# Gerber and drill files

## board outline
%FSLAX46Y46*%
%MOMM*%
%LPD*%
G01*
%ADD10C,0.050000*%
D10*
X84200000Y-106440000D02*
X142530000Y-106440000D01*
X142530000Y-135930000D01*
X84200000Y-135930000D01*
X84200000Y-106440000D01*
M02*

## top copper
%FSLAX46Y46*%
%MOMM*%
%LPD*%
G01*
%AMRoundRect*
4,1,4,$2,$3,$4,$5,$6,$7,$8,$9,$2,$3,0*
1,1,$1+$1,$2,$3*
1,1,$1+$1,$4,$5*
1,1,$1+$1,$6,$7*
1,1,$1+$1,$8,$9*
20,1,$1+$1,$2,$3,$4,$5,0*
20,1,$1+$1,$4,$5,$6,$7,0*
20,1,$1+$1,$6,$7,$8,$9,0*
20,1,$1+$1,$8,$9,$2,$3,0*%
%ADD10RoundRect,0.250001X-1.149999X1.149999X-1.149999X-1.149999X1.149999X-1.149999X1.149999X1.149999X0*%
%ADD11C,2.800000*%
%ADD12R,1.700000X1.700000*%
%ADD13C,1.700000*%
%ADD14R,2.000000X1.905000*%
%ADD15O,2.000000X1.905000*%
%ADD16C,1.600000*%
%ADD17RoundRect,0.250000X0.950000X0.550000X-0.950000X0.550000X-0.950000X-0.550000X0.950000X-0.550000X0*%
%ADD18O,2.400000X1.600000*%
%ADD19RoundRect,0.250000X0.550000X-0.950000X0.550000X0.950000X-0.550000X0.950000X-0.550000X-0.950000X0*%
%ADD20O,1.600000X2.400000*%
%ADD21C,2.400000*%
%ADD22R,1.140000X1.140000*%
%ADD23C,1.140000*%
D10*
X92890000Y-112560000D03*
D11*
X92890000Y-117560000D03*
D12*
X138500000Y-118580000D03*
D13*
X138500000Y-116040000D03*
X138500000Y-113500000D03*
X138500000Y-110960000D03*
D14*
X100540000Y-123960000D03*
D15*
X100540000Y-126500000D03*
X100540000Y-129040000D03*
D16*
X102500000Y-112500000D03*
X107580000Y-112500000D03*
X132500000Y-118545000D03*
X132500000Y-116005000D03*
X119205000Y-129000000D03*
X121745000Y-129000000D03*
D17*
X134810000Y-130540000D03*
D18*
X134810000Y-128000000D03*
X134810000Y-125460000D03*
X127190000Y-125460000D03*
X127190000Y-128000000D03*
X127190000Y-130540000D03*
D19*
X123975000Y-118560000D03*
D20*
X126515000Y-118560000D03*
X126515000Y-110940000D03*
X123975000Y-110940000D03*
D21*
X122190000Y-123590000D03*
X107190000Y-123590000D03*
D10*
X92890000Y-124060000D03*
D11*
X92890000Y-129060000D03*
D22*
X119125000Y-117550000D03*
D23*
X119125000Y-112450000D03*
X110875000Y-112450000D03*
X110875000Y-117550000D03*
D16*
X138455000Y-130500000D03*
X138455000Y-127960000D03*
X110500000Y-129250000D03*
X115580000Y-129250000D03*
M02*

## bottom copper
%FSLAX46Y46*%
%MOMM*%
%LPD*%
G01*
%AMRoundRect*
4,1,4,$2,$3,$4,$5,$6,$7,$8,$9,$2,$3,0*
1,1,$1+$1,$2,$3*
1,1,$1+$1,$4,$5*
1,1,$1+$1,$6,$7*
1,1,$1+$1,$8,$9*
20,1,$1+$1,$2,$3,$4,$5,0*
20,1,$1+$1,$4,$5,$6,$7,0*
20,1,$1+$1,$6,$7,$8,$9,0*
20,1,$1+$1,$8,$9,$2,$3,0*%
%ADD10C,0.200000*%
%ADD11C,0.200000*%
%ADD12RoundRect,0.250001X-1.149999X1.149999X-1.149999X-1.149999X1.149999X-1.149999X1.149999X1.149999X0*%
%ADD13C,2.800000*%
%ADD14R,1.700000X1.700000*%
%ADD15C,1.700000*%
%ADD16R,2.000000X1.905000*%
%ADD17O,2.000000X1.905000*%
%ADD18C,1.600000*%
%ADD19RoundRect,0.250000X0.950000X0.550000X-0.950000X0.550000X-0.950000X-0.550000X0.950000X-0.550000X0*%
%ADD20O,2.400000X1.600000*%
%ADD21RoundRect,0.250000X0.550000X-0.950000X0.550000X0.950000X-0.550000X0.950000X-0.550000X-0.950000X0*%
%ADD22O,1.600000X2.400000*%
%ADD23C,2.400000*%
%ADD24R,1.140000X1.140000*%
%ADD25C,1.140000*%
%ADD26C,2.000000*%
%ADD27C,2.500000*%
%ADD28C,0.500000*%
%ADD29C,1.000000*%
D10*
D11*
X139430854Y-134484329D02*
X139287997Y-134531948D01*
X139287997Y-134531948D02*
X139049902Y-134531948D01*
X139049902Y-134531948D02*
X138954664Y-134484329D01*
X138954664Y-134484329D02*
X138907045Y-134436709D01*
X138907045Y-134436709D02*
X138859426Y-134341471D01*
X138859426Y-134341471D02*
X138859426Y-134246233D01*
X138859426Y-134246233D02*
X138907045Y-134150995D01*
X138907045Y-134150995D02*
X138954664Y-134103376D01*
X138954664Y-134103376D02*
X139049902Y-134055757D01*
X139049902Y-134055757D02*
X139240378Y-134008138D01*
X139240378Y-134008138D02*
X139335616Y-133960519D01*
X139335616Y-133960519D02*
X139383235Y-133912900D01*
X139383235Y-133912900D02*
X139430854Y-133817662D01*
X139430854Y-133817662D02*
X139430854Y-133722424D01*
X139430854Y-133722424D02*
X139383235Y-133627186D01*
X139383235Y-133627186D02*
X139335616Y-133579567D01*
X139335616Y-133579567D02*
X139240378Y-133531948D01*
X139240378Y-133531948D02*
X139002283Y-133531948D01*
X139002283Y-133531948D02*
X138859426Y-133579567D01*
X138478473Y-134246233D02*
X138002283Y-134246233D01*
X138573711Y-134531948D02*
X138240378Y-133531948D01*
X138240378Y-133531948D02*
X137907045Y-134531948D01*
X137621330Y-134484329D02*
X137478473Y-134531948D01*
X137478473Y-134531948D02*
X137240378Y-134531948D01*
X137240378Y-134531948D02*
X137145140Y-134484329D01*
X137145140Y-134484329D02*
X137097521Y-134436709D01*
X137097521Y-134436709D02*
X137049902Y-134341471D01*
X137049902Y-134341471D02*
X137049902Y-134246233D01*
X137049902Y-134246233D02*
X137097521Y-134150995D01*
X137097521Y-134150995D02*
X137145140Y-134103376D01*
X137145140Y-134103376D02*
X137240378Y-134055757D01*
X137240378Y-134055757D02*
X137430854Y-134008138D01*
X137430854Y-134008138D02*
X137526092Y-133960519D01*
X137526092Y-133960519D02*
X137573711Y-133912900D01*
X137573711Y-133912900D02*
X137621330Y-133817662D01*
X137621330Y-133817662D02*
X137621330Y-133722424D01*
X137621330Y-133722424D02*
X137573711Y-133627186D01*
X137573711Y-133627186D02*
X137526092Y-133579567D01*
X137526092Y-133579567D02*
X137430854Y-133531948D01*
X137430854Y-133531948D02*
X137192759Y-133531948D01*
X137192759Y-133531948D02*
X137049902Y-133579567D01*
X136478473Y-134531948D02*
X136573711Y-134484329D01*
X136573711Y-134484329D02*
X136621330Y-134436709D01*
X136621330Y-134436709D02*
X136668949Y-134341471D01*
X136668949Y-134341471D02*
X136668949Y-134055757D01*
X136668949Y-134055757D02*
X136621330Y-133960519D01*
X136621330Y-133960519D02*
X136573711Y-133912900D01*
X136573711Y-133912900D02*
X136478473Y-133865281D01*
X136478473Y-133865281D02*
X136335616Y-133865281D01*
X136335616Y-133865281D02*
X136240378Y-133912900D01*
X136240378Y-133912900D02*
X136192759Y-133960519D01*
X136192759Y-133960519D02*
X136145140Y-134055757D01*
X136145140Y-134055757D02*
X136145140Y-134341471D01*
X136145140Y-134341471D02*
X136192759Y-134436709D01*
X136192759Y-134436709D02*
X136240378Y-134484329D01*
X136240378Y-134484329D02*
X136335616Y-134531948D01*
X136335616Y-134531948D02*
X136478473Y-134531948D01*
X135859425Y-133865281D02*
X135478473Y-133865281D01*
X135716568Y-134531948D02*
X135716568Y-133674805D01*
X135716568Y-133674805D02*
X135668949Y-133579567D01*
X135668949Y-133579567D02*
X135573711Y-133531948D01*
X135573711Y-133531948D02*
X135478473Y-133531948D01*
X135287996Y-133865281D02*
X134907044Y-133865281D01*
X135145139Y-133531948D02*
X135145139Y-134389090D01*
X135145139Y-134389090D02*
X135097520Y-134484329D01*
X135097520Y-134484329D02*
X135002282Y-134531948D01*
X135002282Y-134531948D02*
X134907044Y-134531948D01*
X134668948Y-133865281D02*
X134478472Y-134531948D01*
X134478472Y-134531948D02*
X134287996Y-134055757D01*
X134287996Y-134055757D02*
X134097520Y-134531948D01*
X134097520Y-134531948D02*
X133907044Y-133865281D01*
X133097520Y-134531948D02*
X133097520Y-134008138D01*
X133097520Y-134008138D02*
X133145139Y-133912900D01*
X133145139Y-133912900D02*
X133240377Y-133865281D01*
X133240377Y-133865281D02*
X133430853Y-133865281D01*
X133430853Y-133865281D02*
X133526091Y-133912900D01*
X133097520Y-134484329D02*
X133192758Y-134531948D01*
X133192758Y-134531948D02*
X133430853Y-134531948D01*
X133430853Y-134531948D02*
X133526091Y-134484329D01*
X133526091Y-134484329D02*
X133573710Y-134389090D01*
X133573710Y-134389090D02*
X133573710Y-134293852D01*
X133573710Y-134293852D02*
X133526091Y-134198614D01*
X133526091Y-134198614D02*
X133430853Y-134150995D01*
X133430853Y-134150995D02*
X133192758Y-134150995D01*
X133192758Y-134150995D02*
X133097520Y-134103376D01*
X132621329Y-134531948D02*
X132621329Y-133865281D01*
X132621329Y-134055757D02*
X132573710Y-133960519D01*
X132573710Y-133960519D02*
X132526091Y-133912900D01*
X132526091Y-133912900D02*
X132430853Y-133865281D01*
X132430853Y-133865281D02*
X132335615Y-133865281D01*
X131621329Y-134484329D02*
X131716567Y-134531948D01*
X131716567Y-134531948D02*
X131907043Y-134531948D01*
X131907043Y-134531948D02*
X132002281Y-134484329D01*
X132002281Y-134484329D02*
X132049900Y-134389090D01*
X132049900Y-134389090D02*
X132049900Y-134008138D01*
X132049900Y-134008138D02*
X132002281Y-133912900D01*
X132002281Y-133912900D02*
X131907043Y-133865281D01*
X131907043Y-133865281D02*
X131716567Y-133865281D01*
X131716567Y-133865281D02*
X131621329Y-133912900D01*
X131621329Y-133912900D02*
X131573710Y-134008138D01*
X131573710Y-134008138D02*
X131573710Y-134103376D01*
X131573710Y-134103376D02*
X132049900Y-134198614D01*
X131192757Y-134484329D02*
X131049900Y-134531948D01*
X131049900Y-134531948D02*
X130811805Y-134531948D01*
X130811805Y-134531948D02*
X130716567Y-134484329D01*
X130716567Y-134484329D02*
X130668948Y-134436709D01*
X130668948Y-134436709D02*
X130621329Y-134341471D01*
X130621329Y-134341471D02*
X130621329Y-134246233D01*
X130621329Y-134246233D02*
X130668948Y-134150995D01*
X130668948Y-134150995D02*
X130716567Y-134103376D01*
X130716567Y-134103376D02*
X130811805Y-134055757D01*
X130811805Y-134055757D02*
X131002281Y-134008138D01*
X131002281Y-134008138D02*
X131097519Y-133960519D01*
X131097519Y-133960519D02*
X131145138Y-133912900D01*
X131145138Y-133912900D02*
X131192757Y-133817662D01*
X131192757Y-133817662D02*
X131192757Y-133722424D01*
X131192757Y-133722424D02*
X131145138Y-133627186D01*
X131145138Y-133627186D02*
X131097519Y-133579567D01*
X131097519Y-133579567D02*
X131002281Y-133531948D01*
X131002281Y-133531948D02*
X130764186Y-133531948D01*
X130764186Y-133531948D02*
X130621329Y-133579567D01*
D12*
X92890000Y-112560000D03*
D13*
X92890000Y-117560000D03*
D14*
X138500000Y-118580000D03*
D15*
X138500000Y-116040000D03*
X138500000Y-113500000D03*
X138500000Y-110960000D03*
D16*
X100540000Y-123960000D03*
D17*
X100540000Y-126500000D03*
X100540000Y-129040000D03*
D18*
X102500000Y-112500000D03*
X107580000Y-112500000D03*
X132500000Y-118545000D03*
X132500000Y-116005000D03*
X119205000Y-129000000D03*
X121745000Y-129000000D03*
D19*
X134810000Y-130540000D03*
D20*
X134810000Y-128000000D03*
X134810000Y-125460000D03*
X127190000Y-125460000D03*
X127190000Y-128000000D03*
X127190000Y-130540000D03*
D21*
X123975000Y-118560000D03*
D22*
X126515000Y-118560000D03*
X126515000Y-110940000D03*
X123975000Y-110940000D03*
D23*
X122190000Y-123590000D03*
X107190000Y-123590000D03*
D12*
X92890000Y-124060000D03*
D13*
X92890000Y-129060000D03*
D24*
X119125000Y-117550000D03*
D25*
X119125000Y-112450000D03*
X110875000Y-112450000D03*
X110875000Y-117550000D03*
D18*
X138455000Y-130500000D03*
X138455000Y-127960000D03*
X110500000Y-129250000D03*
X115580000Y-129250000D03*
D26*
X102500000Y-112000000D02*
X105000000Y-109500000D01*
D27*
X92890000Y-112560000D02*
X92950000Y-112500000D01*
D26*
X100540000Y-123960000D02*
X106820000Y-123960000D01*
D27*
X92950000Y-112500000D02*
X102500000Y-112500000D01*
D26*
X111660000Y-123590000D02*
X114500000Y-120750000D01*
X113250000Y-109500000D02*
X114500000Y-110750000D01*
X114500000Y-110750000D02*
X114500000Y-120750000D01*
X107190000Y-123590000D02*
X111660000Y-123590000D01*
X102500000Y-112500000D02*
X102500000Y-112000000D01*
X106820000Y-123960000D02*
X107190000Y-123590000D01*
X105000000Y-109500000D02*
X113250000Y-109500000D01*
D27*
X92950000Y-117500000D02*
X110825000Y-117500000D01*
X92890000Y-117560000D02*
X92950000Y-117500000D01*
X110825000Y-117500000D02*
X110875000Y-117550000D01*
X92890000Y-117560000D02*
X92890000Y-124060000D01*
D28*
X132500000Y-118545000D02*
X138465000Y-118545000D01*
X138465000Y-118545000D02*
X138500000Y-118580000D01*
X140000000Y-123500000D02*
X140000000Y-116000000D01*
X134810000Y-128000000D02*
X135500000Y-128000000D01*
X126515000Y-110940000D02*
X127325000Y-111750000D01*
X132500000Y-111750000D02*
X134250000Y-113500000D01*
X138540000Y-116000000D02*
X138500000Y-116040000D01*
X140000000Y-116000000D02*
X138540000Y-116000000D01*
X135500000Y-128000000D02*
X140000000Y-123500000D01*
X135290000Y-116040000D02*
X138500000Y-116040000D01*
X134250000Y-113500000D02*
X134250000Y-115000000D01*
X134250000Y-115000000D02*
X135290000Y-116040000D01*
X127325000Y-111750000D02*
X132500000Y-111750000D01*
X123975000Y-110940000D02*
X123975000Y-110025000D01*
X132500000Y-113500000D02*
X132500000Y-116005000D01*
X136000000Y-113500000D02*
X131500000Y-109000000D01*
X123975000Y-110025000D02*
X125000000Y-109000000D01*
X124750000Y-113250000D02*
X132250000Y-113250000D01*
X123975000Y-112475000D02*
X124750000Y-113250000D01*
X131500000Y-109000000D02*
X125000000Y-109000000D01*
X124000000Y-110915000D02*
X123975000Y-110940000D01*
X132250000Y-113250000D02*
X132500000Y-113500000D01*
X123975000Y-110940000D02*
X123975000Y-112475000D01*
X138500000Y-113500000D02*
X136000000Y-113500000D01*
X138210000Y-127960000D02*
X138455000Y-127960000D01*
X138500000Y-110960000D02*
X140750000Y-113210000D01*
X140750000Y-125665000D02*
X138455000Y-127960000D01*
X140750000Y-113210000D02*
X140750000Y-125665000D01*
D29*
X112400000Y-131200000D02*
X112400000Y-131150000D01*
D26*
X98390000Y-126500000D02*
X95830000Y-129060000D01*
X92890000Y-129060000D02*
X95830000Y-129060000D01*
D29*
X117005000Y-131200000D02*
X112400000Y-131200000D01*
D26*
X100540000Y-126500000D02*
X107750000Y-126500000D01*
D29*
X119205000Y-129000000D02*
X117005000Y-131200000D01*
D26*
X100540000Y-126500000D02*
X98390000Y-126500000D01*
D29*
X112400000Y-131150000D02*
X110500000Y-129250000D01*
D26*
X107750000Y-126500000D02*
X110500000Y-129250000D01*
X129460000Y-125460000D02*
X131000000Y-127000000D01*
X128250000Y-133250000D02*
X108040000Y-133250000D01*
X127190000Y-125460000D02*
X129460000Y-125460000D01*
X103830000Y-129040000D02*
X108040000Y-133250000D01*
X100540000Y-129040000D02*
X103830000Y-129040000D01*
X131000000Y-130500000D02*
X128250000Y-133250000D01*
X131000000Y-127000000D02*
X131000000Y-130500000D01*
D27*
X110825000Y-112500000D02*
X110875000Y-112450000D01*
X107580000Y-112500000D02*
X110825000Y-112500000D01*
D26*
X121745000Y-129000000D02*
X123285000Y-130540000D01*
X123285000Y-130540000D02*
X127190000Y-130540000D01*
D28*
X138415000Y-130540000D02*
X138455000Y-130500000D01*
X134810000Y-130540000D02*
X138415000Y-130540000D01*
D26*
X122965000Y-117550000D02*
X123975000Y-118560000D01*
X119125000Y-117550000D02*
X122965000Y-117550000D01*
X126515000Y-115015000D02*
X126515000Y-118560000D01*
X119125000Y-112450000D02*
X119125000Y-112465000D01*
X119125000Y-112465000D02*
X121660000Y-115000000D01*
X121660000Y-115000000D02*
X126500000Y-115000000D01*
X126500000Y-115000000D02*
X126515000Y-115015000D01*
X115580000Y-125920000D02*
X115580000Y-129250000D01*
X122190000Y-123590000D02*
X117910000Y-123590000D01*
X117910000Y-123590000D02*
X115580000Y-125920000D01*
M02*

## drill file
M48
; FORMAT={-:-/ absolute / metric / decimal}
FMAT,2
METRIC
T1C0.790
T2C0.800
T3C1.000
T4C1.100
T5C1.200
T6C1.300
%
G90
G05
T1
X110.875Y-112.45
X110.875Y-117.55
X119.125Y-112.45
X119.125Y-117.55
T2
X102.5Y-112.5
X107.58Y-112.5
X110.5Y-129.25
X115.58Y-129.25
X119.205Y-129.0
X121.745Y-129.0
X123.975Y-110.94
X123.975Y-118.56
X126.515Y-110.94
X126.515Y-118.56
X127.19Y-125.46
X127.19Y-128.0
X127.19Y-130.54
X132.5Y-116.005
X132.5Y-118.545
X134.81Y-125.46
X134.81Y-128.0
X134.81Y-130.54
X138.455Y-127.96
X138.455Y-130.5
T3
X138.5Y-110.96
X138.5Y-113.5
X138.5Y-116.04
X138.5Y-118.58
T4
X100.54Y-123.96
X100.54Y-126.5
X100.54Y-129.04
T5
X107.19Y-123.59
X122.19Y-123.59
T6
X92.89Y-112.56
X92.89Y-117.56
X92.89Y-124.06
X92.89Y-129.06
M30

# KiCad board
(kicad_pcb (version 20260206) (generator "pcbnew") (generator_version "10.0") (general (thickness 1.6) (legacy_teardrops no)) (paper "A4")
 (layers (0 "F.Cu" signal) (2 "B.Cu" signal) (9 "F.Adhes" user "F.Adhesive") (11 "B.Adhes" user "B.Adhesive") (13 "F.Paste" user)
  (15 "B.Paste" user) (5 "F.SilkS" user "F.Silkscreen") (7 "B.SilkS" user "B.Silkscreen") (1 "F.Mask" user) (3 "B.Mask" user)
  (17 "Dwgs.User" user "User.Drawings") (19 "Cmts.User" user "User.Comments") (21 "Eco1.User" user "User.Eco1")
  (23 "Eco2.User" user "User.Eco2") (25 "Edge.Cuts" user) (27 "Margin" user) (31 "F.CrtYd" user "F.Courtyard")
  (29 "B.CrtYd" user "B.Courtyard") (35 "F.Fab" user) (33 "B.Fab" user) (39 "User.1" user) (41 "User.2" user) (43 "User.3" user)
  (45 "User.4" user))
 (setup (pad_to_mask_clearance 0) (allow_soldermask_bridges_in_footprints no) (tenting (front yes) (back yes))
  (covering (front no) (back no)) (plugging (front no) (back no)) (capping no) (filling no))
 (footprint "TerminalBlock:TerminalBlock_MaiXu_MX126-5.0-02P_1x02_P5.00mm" (layer "F.Cu") (at 92.89 112.56 -90)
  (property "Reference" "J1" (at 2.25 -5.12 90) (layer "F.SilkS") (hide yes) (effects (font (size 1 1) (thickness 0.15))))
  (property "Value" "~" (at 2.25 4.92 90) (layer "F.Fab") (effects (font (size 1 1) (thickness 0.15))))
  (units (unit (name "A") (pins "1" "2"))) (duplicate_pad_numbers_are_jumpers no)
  (pad "1" thru_hole roundrect (at 0 0 270) (size 2.8 2.8) (drill 1.3) (layers "*.Cu" "*.Mask") (remove_unused_layers no)
   (roundrect_rratio 0.089286) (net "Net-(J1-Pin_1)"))
  (pad "2" thru_hole circle (at 5 0 270) (size 2.8 2.8) (drill 1.3) (layers "*.Cu" "*.Mask") (remove_unused_layers no)
   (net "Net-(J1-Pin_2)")))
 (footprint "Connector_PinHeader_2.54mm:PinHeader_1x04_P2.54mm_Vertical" (layer "F.Cu") (at 138.5 118.58 180)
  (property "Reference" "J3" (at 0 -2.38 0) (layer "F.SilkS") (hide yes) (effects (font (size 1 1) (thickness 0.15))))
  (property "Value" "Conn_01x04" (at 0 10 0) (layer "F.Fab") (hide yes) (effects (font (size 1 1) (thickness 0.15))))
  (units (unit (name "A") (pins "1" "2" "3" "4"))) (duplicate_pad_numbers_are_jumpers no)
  (pad "1" thru_hole rect (at 0 0 180) (size 1.7 1.7) (drill 1) (layers "*.Cu" "*.Mask") (remove_unused_layers no) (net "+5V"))
  (pad "2" thru_hole circle (at 0 2.54 180) (size 1.7 1.7) (drill 1) (layers "*.Cu" "*.Mask") (remove_unused_layers no) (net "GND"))
  (pad "3" thru_hole circle (at 0 5.08 180) (size 1.7 1.7) (drill 1) (layers "*.Cu" "*.Mask") (remove_unused_layers no)
   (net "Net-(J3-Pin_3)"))
  (pad "4" thru_hole circle (at 0 7.62 180) (size 1.7 1.7) (drill 1) (layers "*.Cu" "*.Mask") (remove_unused_layers no)
   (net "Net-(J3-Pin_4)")))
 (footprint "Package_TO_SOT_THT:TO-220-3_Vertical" (layer "F.Cu") (at 100.54 123.96 -90)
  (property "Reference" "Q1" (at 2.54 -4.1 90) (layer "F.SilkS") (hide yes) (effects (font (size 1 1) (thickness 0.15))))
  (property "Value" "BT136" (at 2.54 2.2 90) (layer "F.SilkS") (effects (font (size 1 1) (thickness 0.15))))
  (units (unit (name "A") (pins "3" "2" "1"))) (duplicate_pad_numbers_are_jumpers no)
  (pad "1" thru_hole rect (at 0 0 270) (size 1.905 2) (drill 1.1) (layers "*.Cu" "*.Mask") (remove_unused_layers no) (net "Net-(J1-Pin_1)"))
  (pad "2" thru_hole oval (at 2.54 0 270) (size 1.905 2) (drill 1.1) (layers "*.Cu" "*.Mask") (remove_unused_layers no)
   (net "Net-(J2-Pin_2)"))
  (pad "3" thru_hole oval (at 5.08 0 270) (size 1.905 2) (drill 1.1) (layers "*.Cu" "*.Mask") (remove_unused_layers no) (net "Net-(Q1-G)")))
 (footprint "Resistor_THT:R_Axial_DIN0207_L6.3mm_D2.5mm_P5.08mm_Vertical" (layer "F.Cu") (at 102.5 112.5)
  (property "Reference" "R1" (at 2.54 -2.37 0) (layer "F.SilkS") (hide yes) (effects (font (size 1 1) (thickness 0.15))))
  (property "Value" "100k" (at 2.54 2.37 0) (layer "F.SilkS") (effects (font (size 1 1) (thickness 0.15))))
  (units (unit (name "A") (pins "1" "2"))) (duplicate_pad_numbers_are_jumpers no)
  (pad "1" thru_hole circle (at 0 0) (size 1.6 1.6) (drill 0.8) (layers "*.Cu" "*.Mask") (remove_unused_layers no) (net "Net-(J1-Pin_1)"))
  (pad "2" thru_hole circle (at 5.08 0) (size 1.6 1.6) (drill 0.8) (layers "*.Cu" "*.Mask") (remove_unused_layers no) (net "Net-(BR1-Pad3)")))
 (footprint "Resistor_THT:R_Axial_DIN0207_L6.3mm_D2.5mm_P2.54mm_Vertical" (layer "F.Cu") (at 132.5 118.545 90)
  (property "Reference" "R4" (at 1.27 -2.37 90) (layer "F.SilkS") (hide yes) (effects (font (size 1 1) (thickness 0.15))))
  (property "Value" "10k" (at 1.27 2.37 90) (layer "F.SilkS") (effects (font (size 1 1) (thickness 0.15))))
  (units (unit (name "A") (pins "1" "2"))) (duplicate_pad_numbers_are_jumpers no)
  (pad "1" thru_hole circle (at 0 0 90) (size 1.6 1.6) (drill 0.8) (layers "*.Cu" "*.Mask") (remove_unused_layers no) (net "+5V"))
  (pad "2" thru_hole circle (at 2.54 0 90) (size 1.6 1.6) (drill 0.8) (layers "*.Cu" "*.Mask") (remove_unused_layers no)
   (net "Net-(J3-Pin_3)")))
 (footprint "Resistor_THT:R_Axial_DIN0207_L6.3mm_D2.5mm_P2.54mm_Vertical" (layer "F.Cu") (at 119.205 129)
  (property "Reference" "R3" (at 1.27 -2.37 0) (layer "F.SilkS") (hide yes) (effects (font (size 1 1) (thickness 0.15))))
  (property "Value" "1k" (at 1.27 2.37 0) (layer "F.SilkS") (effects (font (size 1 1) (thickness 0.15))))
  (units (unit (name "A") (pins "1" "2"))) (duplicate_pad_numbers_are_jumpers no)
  (pad "1" thru_hole circle (at 0 0) (size 1.6 1.6) (drill 0.8) (layers "*.Cu" "*.Mask") (remove_unused_layers no) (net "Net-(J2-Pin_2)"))
  (pad "2" thru_hole circle (at 2.54 0) (size 1.6 1.6) (drill 0.8) (layers "*.Cu" "*.Mask") (remove_unused_layers no) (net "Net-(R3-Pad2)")))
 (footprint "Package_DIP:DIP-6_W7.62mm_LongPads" (layer "F.Cu") (at 134.81 130.54 180)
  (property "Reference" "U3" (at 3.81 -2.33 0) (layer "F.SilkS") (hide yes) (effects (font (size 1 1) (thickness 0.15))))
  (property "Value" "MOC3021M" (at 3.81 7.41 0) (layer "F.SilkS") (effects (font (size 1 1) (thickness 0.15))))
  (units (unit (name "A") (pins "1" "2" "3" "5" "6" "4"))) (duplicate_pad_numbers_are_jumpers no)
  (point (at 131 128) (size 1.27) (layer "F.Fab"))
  (pad "1" thru_hole roundrect (at 0 0 180) (size 2.4 1.6) (drill 0.8) (layers "*.Cu" "*.Mask") (remove_unused_layers no)
   (roundrect_rratio 0.15625) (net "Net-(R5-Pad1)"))
  (pad "2" thru_hole oval (at 0 2.54 180) (size 2.4 1.6) (drill 0.8) (layers "*.Cu" "*.Mask") (remove_unused_layers no) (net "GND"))
  (pad "3" thru_hole oval (at 0 5.08 180) (size 2.4 1.6) (drill 0.8) (layers "*.Cu" "*.Mask") (remove_unused_layers no)
   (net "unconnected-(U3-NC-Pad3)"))
  (pad "4" thru_hole oval (at 7.62 5.08 180) (size 2.4 1.6) (drill 0.8) (layers "*.Cu" "*.Mask") (remove_unused_layers no)
   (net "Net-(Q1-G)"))
  (pad "5" thru_hole oval (at 7.62 2.54 180) (size 2.4 1.6) (drill 0.8) (layers "*.Cu" "*.Mask") (remove_unused_layers no)
   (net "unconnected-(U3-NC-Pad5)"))
  (pad "6" thru_hole oval (at 7.62 0 180) (size 2.4 1.6) (drill 0.8) (layers "*.Cu" "*.Mask") (remove_unused_layers no)
   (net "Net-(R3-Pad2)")))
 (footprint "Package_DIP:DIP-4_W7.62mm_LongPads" (layer "F.Cu") (at 123.975 118.56 90)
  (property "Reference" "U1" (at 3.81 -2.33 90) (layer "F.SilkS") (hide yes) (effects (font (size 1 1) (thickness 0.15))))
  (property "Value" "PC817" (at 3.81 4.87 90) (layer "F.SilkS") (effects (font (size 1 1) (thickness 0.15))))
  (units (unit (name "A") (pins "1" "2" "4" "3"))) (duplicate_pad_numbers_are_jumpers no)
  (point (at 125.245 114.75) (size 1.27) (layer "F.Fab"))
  (pad "1" thru_hole roundrect (at 0 0 90) (size 2.4 1.6) (drill 0.8) (layers "*.Cu" "*.Mask") (remove_unused_layers no)
   (roundrect_rratio 0.15625) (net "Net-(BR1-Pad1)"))
  (pad "2" thru_hole oval (at 0 2.54 90) (size 2.4 1.6) (drill 0.8) (layers "*.Cu" "*.Mask") (remove_unused_layers no)
   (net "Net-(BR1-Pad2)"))
  (pad "3" thru_hole oval (at 7.62 2.54 90) (size 2.4 1.6) (drill 0.8) (layers "*.Cu" "*.Mask") (remove_unused_layers no) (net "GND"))
  (pad "4" thru_hole oval (at 7.62 0 90) (size 2.4 1.6) (drill 0.8) (layers "*.Cu" "*.Mask") (remove_unused_layers no)
   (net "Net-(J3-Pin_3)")))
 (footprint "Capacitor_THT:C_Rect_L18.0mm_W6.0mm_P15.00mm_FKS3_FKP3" (layer "F.Cu") (at 122.19 123.59 180)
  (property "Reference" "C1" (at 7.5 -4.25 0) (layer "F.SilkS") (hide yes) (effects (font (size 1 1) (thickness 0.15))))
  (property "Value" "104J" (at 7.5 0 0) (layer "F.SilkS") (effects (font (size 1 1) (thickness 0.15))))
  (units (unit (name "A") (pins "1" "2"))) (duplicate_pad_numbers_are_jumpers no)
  (pad "1" thru_hole circle (at 0 0 180) (size 2.4 2.4) (drill 1.2) (layers "*.Cu" "*.Mask") (remove_unused_layers no) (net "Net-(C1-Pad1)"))
  (pad "2" thru_hole circle (at 15 0 180) (size 2.4 2.4) (drill 1.2) (layers "*.Cu" "*.Mask") (remove_unused_layers no)
   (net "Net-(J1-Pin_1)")))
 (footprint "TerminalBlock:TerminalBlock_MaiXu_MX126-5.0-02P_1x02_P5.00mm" (layer "F.Cu") (at 92.89 124.06 -90)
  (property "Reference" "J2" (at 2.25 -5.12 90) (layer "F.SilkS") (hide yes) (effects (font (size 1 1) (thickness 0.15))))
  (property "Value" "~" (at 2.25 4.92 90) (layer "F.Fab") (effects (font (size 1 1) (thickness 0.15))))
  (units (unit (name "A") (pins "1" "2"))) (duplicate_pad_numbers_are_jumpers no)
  (pad "1" thru_hole roundrect (at 0 0 270) (size 2.8 2.8) (drill 1.3) (layers "*.Cu" "*.Mask") (remove_unused_layers no)
   (roundrect_rratio 0.089286) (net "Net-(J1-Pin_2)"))
  (pad "2" thru_hole circle (at 5 0 270) (size 2.8 2.8) (drill 1.3) (layers "*.Cu" "*.Mask") (remove_unused_layers no)
   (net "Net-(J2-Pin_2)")))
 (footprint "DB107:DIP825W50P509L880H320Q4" (layer "F.Cu") (at 115 115 180)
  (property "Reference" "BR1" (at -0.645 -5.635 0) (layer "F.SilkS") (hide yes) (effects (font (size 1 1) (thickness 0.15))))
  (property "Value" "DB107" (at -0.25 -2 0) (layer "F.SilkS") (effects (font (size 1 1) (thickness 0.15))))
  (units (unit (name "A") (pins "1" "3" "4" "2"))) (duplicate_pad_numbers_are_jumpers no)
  (pad "1" thru_hole rect (at -4.125 -2.55 180) (size 1.14 1.14) (drill 0.79) (layers "*.Cu" "*.Mask") (remove_unused_layers no)
   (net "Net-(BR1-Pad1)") (solder_mask_margin 0.102))
  (pad "2" thru_hole circle (at -4.125 2.55 180) (size 1.14 1.14) (drill 0.79) (layers "*.Cu" "*.Mask") (remove_unused_layers no)
   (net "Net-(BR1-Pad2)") (solder_mask_margin 0.102))
  (pad "3" thru_hole circle (at 4.125 2.55 180) (size 1.14 1.14) (drill 0.79) (layers "*.Cu" "*.Mask") (remove_unused_layers no)
   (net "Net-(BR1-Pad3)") (solder_mask_margin 0.102))
  (pad "4" thru_hole circle (at 4.125 -2.55 180) (size 1.14 1.14) (drill 0.79) (layers "*.Cu" "*.Mask") (remove_unused_layers no)
   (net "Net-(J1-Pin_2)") (solder_mask_margin 0.102)))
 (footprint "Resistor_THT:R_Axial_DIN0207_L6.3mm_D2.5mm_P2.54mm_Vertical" (layer "F.Cu") (at 138.455 130.5 90)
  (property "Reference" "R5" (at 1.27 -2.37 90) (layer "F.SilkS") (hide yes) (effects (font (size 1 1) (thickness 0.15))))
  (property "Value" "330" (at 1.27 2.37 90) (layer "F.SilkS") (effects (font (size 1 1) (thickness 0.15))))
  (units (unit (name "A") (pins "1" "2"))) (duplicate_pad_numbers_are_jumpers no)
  (pad "1" thru_hole circle (at 0 0 90) (size 1.6 1.6) (drill 0.8) (layers "*.Cu" "*.Mask") (remove_unused_layers no) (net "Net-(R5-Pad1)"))
  (pad "2" thru_hole circle (at 2.54 0 90) (size 1.6 1.6) (drill 0.8) (layers "*.Cu" "*.Mask") (remove_unused_layers no)
   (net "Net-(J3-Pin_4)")))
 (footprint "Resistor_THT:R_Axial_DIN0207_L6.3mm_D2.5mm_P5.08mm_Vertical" (layer "F.Cu") (at 110.5 129.25)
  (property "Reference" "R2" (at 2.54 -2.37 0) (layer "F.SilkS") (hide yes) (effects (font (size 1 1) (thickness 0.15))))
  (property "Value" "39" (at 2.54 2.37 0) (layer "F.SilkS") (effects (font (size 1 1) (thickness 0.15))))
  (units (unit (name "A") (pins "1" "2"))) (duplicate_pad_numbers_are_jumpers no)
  (pad "1" thru_hole circle (at 0 0) (size 1.6 1.6) (drill 0.8) (layers "*.Cu" "*.Mask") (remove_unused_layers no) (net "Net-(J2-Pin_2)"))
  (pad "2" thru_hole circle (at 5.08 0) (size 1.6 1.6) (drill 0.8) (layers "*.Cu" "*.Mask") (remove_unused_layers no) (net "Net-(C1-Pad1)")))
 (gr_rect (start 84.2 106.44) (end 142.53 135.93) (stroke (width 0.05) (type default)) (fill no) (layer "Edge.Cuts"))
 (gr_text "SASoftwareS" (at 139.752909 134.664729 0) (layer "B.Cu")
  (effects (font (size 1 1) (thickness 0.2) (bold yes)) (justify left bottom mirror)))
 (segment (start 102.5 112) (end 105 109.5) (width 2) (layer "B.Cu") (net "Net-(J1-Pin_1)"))
 (segment (start 92.89 112.56) (end 92.95 112.5) (width 2.5) (layer "B.Cu") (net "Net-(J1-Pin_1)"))
 (segment (start 100.54 123.96) (end 106.82 123.96) (width 2) (layer "B.Cu") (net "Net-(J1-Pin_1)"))
 (segment (start 92.95 112.5) (end 102.5 112.5) (width 2.5) (layer "B.Cu") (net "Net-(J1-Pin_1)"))
 (segment (start 111.66 123.59) (end 114.5 120.75) (width 2) (layer "B.Cu") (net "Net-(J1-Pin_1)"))
 (segment (start 113.25 109.5) (end 114.5 110.75) (width 2) (layer "B.Cu") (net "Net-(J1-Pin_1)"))
 (segment (start 114.5 110.75) (end 114.5 120.75) (width 2) (layer "B.Cu") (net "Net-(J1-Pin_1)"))
 (segment (start 107.19 123.59) (end 111.66 123.59) (width 2) (layer "B.Cu") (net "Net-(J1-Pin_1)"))
 (segment (start 102.5 112.5) (end 102.5 112) (width 2) (layer "B.Cu") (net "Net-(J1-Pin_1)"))
 (segment (start 106.82 123.96) (end 107.19 123.59) (width 2) (layer "B.Cu") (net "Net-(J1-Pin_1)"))
 (segment (start 105 109.5) (end 113.25 109.5) (width 2) (layer "B.Cu") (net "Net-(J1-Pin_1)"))
 (segment (start 92.95 117.5) (end 110.825 117.5) (width 2.5) (layer "B.Cu") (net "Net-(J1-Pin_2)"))
 (segment (start 92.89 117.56) (end 92.95 117.5) (width 2.5) (layer "B.Cu") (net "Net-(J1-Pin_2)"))
 (segment (start 110.825 117.5) (end 110.875 117.55) (width 2.5) (layer "B.Cu") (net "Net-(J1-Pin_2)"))
 (segment (start 92.89 117.56) (end 92.89 124.06) (width 2.5) (layer "B.Cu") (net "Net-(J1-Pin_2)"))
 (segment (start 132.5 118.545) (end 138.465 118.545) (width 0.5) (layer "B.Cu") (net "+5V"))
 (segment (start 138.465 118.545) (end 138.5 118.58) (width 0.5) (layer "B.Cu") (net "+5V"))
 (segment (start 140 123.5) (end 140 116) (width 0.5) (layer "B.Cu") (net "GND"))
 (segment (start 134.81 128) (end 135.5 128) (width 0.5) (layer "B.Cu") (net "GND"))
 (segment (start 126.515 110.94) (end 127.325 111.75) (width 0.5) (layer "B.Cu") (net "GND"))
 (segment (start 132.5 111.75) (end 134.25 113.5) (width 0.5) (layer "B.Cu") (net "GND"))
 (segment (start 138.54 116) (end 138.5 116.04) (width 0.5) (layer "B.Cu") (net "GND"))
 (segment (start 140 116) (end 138.54 116) (width 0.5) (layer "B.Cu") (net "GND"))
 (segment (start 135.5 128) (end 140 123.5) (width 0.5) (layer "B.Cu") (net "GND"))
 (segment (start 135.29 116.04) (end 138.5 116.04) (width 0.5) (layer "B.Cu") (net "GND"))
 (segment (start 134.25 113.5) (end 134.25 115) (width 0.5) (layer "B.Cu") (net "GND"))
 (segment (start 134.25 115) (end 135.29 116.04) (width 0.5) (layer "B.Cu") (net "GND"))
 (segment (start 127.325 111.75) (end 132.5 111.75) (width 0.5) (layer "B.Cu") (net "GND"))
 (segment (start 123.975 110.94) (end 123.975 110.025) (width 0.5) (layer "B.Cu") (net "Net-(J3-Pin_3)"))
 (segment (start 132.5 113.5) (end 132.5 116.005) (width 0.5) (layer "B.Cu") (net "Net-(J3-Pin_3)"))
 (segment (start 136 113.5) (end 131.5 109) (width 0.5) (layer "B.Cu") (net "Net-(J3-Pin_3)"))
 (segment (start 123.975 110.025) (end 125 109) (width 0.5) (layer "B.Cu") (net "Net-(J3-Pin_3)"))
 (segment (start 124.75 113.25) (end 132.25 113.25) (width 0.5) (layer "B.Cu") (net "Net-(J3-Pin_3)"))
 (segment (start 123.975 112.475) (end 124.75 113.25) (width 0.5) (layer "B.Cu") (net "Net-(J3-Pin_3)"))
 (segment (start 131.5 109) (end 125 109) (width 0.5) (layer "B.Cu") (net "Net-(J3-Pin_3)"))
 (segment (start 124 110.915) (end 123.975 110.94) (width 0.5) (layer "B.Cu") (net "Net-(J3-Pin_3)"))
 (segment (start 132.25 113.25) (end 132.5 113.5) (width 0.5) (layer "B.Cu") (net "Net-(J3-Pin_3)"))
 (segment (start 123.975 110.94) (end 123.975 112.475) (width 0.5) (layer "B.Cu") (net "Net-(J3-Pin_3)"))
 (segment (start 138.5 113.5) (end 136 113.5) (width 0.5) (layer "B.Cu") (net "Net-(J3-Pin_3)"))
 (segment (start 138.21 127.96) (end 138.455 127.96) (width 0.5) (layer "B.Cu") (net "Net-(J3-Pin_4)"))
 (segment (start 138.5 110.96) (end 140.75 113.21) (width 0.5) (layer "B.Cu") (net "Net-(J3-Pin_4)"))
 (segment (start 140.75 125.665) (end 138.455 127.96) (width 0.5) (layer "B.Cu") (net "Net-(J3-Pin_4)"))
 (segment (start 140.75 113.21) (end 140.75 125.665) (width 0.5) (layer "B.Cu") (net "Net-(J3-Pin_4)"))
 (segment (start 112.4 131.2) (end 112.4 131.15) (width 1) (layer "B.Cu") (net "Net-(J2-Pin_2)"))
 (segment (start 98.39 126.5) (end 95.83 129.06) (width 2) (layer "B.Cu") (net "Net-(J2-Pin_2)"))
 (segment (start 92.89 129.06) (end 95.83 129.06) (width 2) (layer "B.Cu") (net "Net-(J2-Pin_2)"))
 (segment (start 117.005 131.2) (end 112.4 131.2) (width 1) (layer "B.Cu") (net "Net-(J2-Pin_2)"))
 (segment (start 100.54 126.5) (end 107.75 126.5) (width 2) (layer "B.Cu") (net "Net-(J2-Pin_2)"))
 (segment (start 119.205 129) (end 117.005 131.2) (width 1) (layer "B.Cu") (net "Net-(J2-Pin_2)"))
 (segment (start 100.54 126.5) (end 98.39 126.5) (width 2) (layer "B.Cu") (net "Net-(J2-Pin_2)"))
 (segment (start 112.4 131.15) (end 110.5 129.25) (width 1) (layer "B.Cu") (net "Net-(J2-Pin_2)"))
 (segment (start 107.75 126.5) (end 110.5 129.25) (width 2) (layer "B.Cu") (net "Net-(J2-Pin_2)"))
 (segment (start 129.46 125.46) (end 131 127) (width 2) (layer "B.Cu") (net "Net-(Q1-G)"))
 (segment (start 128.25 133.25) (end 108.04 133.25) (width 2) (layer "B.Cu") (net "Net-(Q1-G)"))
 (segment (start 127.19 125.46) (end 129.46 125.46) (width 2) (layer "B.Cu") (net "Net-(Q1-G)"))
 (segment (start 103.83 129.04) (end 108.04 133.25) (width 2) (layer "B.Cu") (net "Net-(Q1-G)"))
 (segment (start 100.54 129.04) (end 103.83 129.04) (width 2) (layer "B.Cu") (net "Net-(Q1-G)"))
 (segment (start 131 130.5) (end 128.25 133.25) (width 2) (layer "B.Cu") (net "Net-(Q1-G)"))
 (segment (start 131 127) (end 131 130.5) (width 2) (layer "B.Cu") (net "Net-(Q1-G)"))
 (segment (start 110.825 112.5) (end 110.875 112.45) (width 2.5) (layer "B.Cu") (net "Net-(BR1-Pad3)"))
 (segment (start 107.58 112.5) (end 110.825 112.5) (width 2.5) (layer "B.Cu") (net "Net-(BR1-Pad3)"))
 (segment (start 121.745 129) (end 123.285 130.54) (width 2) (layer "B.Cu") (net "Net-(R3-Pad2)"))
 (segment (start 123.285 130.54) (end 127.19 130.54) (width 2) (layer "B.Cu") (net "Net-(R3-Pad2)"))
 (segment (start 138.415 130.54) (end 138.455 130.5) (width 0.5) (layer "B.Cu") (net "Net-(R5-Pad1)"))
 (segment (start 134.81 130.54) (end 138.415 130.54) (width 0.5) (layer "B.Cu") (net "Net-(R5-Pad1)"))
 (segment (start 122.965 117.55) (end 123.975 118.56) (width 2) (layer "B.Cu") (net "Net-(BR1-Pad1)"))
 (segment (start 119.125 117.55) (end 122.965 117.55) (width 2) (layer "B.Cu") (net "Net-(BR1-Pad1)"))
 (segment (start 126.515 115.015) (end 126.515 118.56) (width 2) (layer "B.Cu") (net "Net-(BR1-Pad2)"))
 (segment (start 119.125 112.45) (end 119.125 112.465) (width 2) (layer "B.Cu") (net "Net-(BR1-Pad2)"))
 (segment (start 119.125 112.465) (end 121.66 115) (width 2) (layer "B.Cu") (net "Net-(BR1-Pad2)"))
 (segment (start 121.66 115) (end 126.5 115) (width 2) (layer "B.Cu") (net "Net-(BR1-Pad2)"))
 (segment (start 126.5 115) (end 126.515 115.015) (width 2) (layer "B.Cu") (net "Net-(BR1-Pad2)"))
 (segment (start 115.58 125.92) (end 115.58 129.25) (width 2) (layer "B.Cu") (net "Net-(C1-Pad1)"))
 (segment (start 122.19 123.59) (end 117.91 123.59) (width 2) (layer "B.Cu") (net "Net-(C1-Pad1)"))
 (segment (start 117.91 123.59) (end 115.58 125.92) (width 2) (layer "B.Cu") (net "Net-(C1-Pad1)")))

